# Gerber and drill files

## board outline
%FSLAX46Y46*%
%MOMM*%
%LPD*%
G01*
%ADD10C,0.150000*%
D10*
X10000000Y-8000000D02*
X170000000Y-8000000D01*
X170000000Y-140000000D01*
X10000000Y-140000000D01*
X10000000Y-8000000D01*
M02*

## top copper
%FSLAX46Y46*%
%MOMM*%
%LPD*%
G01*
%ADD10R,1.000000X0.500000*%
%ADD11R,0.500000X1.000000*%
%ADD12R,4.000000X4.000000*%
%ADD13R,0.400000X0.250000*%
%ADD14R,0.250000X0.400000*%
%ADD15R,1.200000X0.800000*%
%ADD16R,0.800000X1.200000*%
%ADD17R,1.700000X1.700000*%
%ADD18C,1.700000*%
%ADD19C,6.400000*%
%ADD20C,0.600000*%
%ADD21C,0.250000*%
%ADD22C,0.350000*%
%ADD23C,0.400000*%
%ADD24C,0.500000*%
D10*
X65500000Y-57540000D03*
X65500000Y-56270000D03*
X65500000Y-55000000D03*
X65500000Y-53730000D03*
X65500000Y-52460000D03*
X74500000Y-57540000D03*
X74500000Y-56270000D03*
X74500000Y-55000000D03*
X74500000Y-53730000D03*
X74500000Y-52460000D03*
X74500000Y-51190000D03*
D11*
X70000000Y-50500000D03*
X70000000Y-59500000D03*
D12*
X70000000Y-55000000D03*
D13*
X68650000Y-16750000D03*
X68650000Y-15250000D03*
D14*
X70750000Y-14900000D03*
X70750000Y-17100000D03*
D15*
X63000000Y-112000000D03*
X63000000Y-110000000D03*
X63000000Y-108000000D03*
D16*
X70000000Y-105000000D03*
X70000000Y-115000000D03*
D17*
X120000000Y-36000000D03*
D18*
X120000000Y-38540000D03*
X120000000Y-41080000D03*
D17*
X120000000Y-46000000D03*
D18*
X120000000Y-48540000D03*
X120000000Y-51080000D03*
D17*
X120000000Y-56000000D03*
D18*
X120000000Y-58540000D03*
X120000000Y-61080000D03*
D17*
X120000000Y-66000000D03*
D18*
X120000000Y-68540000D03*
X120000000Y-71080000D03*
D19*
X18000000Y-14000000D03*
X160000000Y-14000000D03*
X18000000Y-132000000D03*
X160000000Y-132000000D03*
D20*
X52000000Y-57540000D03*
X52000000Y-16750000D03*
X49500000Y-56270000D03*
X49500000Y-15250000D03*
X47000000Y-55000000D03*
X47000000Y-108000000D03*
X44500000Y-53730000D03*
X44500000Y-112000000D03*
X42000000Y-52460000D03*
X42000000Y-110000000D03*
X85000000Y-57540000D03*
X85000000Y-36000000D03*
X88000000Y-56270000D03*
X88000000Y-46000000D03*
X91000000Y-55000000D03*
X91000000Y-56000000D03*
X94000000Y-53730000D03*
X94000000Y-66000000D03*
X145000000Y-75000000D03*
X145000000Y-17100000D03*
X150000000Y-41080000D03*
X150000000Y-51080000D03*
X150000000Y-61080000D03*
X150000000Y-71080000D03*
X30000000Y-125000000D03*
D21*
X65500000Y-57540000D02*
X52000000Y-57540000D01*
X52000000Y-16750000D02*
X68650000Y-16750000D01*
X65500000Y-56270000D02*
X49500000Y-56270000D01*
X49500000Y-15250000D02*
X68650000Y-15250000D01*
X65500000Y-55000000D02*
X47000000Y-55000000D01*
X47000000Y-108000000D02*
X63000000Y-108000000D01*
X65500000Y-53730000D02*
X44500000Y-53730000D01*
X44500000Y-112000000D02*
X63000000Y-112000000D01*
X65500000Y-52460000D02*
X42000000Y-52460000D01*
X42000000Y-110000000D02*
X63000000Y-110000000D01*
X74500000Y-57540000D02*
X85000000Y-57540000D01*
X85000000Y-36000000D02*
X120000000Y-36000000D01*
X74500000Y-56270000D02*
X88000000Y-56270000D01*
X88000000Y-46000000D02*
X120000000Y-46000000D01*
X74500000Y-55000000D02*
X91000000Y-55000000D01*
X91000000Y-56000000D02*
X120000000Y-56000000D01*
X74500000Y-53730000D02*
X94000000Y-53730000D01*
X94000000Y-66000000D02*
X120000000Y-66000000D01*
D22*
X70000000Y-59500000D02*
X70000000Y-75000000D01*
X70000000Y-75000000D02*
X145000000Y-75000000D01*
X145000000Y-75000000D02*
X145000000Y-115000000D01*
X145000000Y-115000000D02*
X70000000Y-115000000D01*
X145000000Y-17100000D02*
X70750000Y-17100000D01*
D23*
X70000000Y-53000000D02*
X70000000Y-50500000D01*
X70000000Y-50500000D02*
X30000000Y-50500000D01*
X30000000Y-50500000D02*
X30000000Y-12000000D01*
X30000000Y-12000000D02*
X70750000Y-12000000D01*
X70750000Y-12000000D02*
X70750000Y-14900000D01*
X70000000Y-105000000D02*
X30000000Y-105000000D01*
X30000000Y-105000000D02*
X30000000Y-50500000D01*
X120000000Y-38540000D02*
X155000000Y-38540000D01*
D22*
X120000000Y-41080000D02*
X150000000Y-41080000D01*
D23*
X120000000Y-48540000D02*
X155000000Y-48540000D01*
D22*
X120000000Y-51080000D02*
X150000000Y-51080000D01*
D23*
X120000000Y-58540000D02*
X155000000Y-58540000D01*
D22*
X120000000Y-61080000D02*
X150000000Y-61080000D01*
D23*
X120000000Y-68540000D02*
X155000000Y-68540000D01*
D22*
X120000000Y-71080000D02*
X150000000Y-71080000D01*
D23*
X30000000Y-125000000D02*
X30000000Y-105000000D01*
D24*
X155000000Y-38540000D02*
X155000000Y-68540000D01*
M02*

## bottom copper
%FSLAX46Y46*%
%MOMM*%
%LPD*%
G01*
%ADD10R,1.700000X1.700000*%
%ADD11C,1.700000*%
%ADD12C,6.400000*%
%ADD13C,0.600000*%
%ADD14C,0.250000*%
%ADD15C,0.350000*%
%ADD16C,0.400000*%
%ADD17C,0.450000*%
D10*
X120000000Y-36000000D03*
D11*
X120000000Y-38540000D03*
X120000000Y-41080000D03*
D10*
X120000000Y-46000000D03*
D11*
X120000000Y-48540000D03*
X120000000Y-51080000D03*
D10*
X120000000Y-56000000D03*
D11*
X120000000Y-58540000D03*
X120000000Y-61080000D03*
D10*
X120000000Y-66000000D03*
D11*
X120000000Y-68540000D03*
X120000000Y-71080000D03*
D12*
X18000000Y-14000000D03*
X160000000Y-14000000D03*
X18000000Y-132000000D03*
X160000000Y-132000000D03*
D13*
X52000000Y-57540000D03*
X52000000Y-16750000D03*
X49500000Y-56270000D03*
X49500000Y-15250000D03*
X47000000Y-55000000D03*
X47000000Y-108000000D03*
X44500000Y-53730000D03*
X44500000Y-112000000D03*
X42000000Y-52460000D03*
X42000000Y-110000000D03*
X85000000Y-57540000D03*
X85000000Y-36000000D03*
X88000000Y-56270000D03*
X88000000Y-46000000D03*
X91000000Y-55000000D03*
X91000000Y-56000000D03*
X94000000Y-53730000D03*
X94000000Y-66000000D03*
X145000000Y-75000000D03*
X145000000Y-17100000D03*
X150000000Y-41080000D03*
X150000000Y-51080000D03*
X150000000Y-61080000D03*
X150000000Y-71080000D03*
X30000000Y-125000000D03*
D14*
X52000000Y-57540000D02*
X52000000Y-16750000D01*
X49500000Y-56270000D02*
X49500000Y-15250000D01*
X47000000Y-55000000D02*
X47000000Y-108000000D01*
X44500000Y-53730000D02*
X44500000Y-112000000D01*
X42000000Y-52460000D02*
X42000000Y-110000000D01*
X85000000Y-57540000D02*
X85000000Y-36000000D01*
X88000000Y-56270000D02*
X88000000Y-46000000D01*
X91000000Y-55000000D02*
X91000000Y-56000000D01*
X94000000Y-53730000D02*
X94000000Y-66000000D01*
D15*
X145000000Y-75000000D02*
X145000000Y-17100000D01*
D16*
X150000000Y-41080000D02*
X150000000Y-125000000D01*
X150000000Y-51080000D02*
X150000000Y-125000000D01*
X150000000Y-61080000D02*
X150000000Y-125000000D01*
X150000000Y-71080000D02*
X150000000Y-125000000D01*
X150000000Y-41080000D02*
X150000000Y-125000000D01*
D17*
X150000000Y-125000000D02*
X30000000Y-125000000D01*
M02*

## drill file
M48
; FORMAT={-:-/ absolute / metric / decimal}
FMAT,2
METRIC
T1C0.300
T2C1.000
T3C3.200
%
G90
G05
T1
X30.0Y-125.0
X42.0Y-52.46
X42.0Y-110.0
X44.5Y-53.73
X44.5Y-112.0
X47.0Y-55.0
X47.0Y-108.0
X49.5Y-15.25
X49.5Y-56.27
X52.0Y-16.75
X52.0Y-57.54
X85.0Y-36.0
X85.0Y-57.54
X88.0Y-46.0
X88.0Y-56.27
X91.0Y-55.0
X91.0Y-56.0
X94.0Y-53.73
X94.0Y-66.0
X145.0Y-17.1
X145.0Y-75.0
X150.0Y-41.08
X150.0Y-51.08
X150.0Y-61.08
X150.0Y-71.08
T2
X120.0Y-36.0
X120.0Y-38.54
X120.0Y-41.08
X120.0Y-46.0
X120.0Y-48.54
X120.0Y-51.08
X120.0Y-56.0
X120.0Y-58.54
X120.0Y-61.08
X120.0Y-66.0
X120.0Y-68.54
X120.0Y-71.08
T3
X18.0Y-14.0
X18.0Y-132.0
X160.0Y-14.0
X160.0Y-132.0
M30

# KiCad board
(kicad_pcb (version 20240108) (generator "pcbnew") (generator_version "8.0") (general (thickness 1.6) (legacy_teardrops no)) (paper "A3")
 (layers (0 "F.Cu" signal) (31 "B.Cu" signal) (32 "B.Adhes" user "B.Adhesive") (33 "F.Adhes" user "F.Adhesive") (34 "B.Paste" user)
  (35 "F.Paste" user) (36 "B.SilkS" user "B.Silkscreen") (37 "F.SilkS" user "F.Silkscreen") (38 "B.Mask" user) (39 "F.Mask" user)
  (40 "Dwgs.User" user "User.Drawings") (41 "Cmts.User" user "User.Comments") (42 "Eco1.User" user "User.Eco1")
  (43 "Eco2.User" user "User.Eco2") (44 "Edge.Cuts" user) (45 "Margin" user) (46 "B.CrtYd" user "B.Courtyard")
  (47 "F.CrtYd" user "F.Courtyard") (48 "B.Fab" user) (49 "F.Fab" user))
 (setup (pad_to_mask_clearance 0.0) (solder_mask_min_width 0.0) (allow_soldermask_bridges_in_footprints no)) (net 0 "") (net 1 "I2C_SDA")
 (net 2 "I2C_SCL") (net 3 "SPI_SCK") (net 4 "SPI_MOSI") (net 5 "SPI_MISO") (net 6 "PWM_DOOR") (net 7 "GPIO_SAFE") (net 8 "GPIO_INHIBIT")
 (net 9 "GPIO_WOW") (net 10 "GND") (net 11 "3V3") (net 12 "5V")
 (gr_rect (start 10 8) (end 170 140) (stroke (width 0.15) (type solid)) (fill none) (layer "Edge.Cuts"))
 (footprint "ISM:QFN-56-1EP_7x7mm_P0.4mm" (layer "F.Cu") (at 70 55)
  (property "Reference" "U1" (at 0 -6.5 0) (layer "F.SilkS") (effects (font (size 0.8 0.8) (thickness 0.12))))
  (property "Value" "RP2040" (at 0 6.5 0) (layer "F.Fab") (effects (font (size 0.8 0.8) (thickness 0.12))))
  (pad "1" smd rect (at -4.5 2.54) (size 1.0 0.5) (layers "F.Cu" "F.Paste" "F.Mask") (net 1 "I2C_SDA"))
  (pad "2" smd rect (at -4.5 1.27) (size 1.0 0.5) (layers "F.Cu" "F.Paste" "F.Mask") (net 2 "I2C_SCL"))
  (pad "3" smd rect (at -4.5 0) (size 1.0 0.5) (layers "F.Cu" "F.Paste" "F.Mask") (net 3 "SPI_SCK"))
  (pad "4" smd rect (at -4.5 -1.27) (size 1.0 0.5) (layers "F.Cu" "F.Paste" "F.Mask") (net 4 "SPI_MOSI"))
  (pad "5" smd rect (at -4.5 -2.54) (size 1.0 0.5) (layers "F.Cu" "F.Paste" "F.Mask") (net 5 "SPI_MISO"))
  (pad "6" smd rect (at 4.5 2.54) (size 1.0 0.5) (layers "F.Cu" "F.Paste" "F.Mask") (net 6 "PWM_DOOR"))
  (pad "7" smd rect (at 4.5 1.27) (size 1.0 0.5) (layers "F.Cu" "F.Paste" "F.Mask") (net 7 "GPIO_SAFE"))
  (pad "8" smd rect (at 4.5 0) (size 1.0 0.5) (layers "F.Cu" "F.Paste" "F.Mask") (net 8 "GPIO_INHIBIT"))
  (pad "9" smd rect (at 4.5 -1.27) (size 1.0 0.5) (layers "F.Cu" "F.Paste" "F.Mask") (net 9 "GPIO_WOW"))
  (pad "12" smd rect (at 4.5 -2.54) (size 1.0 0.5) (layers "F.Cu" "F.Paste" "F.Mask"))
  (pad "13" smd rect (at 4.5 -3.81) (size 1.0 0.5) (layers "F.Cu" "F.Paste" "F.Mask"))
  (pad "10" smd rect (at 0 -4.5) (size 0.5 1.0) (layers "F.Cu" "F.Paste" "F.Mask") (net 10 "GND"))
  (pad "11" smd rect (at 0 4.5) (size 0.5 1.0) (layers "F.Cu" "F.Paste" "F.Mask") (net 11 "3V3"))
  (pad "EP" smd rect (at 0 0) (size 4 4) (layers "F.Cu" "F.Paste" "F.Mask") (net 10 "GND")))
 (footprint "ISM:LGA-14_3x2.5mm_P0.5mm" (layer "F.Cu") (at 70 16)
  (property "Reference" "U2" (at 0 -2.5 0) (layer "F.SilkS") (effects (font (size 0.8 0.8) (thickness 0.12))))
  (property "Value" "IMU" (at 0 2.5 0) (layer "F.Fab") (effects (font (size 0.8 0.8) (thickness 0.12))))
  (pad "1" smd rect (at -1.35 0.75) (size 0.4 0.25) (layers "F.Cu" "F.Paste" "F.Mask") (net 1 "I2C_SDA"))
  (pad "2" smd rect (at -1.35 -0.75) (size 0.4 0.25) (layers "F.Cu" "F.Paste" "F.Mask") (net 2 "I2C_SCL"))
  (pad "3" smd rect (at 0.75 -1.1) (size 0.25 0.4) (layers "F.Cu" "F.Paste" "F.Mask") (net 10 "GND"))
  (pad "4" smd rect (at 0.75 1.1) (size 0.25 0.4) (layers "F.Cu" "F.Paste" "F.Mask") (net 11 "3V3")))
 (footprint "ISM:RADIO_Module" (layer "F.Cu") (at 70 110)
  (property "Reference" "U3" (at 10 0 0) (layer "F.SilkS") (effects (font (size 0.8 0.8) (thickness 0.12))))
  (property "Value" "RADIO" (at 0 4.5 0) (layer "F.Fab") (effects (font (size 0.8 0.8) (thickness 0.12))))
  (pad "1" smd rect (at -7 2) (size 1.2 0.8) (layers "F.Cu" "F.Paste" "F.Mask") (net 4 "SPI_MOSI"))
  (pad "2" smd rect (at -7 0) (size 1.2 0.8) (layers "F.Cu" "F.Paste" "F.Mask") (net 5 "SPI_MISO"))
  (pad "3" smd rect (at -7 -2) (size 1.2 0.8) (layers "F.Cu" "F.Paste" "F.Mask") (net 3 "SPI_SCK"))
  (pad "4" smd rect (at 0 -5) (size 0.8 1.2) (layers "F.Cu" "F.Paste" "F.Mask") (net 10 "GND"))
  (pad "5" smd rect (at 0 5) (size 0.8 1.2) (layers "F.Cu" "F.Paste" "F.Mask") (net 11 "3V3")))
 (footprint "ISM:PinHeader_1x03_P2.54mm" (layer "F.Cu") (at 120 36)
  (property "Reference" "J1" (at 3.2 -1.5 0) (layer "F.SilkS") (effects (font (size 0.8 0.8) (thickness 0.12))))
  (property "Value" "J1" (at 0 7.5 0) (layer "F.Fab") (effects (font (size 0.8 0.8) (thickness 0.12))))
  (pad "1" thru_hole rect (at 0 0) (size 1.7 1.7) (drill 1.0) (layers "*.Cu" "*.Mask") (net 6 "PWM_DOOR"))
  (pad "2" thru_hole circle (at 0 2.54) (size 1.7 1.7) (drill 1.0) (layers "*.Cu" "*.Mask") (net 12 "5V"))
  (pad "3" thru_hole circle (at 0 5.08) (size 1.7 1.7) (drill 1.0) (layers "*.Cu" "*.Mask") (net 10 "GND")))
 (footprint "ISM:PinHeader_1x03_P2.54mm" (layer "F.Cu") (at 120 46)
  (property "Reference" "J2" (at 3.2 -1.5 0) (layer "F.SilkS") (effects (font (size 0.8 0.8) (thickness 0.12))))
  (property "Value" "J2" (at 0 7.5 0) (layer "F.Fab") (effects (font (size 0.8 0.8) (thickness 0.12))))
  (pad "1" thru_hole rect (at 0 0) (size 1.7 1.7) (drill 1.0) (layers "*.Cu" "*.Mask") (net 7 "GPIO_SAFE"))
  (pad "2" thru_hole circle (at 0 2.54) (size 1.7 1.7) (drill 1.0) (layers "*.Cu" "*.Mask") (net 12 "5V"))
  (pad "3" thru_hole circle (at 0 5.08) (size 1.7 1.7) (drill 1.0) (layers "*.Cu" "*.Mask") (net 10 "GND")))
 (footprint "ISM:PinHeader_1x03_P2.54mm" (layer "F.Cu") (at 120 56)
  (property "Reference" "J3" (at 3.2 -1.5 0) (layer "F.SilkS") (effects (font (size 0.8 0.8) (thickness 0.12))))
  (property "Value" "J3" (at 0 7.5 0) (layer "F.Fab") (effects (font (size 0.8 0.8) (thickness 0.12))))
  (pad "1" thru_hole rect (at 0 0) (size 1.7 1.7) (drill 1.0) (layers "*.Cu" "*.Mask") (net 8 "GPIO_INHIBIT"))
  (pad "2" thru_hole circle (at 0 2.54) (size 1.7 1.7) (drill 1.0) (layers "*.Cu" "*.Mask") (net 12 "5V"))
  (pad "3" thru_hole circle (at 0 5.08) (size 1.7 1.7) (drill 1.0) (layers "*.Cu" "*.Mask") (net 10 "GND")))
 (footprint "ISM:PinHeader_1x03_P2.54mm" (layer "F.Cu") (at 120 66)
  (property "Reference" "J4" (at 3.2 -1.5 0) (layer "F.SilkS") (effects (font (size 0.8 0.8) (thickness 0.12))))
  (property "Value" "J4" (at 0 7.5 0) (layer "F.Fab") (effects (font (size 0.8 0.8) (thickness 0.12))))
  (pad "1" thru_hole rect (at 0 0) (size 1.7 1.7) (drill 1.0) (layers "*.Cu" "*.Mask") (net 9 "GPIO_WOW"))
  (pad "2" thru_hole circle (at 0 2.54) (size 1.7 1.7) (drill 1.0) (layers "*.Cu" "*.Mask") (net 12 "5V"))
  (pad "3" thru_hole circle (at 0 5.08) (size 1.7 1.7) (drill 1.0) (layers "*.Cu" "*.Mask") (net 10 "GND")))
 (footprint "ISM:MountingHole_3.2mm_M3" (layer "F.Cu") (at 18 14)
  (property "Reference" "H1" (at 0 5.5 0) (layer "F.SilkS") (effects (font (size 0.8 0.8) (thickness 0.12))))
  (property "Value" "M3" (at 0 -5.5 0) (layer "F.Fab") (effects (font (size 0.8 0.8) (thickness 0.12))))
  (pad "" thru_hole circle (at 0 0) (size 6.4 6.4) (drill 3.2) (layers "*.Cu" "*.Mask")))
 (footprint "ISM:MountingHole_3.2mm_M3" (layer "F.Cu") (at 160 14)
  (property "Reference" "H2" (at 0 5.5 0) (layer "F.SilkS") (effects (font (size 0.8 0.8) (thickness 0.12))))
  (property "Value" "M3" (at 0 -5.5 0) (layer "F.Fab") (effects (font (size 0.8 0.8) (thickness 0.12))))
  (pad "" thru_hole circle (at 0 0) (size 6.4 6.4) (drill 3.2) (layers "*.Cu" "*.Mask")))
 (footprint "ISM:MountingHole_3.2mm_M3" (layer "F.Cu") (at 18 132)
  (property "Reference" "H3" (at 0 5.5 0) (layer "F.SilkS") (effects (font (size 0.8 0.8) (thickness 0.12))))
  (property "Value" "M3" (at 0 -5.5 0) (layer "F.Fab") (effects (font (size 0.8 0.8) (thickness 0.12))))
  (pad "" thru_hole circle (at 0 0) (size 6.4 6.4) (drill 3.2) (layers "*.Cu" "*.Mask")))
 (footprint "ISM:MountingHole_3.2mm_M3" (layer "F.Cu") (at 160 132)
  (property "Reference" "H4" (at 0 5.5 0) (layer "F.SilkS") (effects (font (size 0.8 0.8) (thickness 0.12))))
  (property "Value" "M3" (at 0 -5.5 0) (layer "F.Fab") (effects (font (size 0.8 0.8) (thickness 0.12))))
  (pad "" thru_hole circle (at 0 0) (size 6.4 6.4) (drill 3.2) (layers "*.Cu" "*.Mask")))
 (segment (start 65.5 57.54) (end 52.0 57.54) (width 0.25) (layer "F.Cu") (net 1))
 (segment (start 52.0 57.54) (end 52.0 16.75) (width 0.25) (layer "B.Cu") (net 1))
 (segment (start 52.0 16.75) (end 68.65 16.75) (width 0.25) (layer "F.Cu") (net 1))
 (segment (start 65.5 56.27) (end 49.5 56.27) (width 0.25) (layer "F.Cu") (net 2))
 (segment (start 49.5 56.27) (end 49.5 15.25) (width 0.25) (layer "B.Cu") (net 2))
 (segment (start 49.5 15.25) (end 68.65 15.25) (width 0.25) (layer "F.Cu") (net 2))
 (segment (start 65.5 55) (end 47.0 55) (width 0.25) (layer "F.Cu") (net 3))
 (segment (start 47.0 55) (end 47.0 108) (width 0.25) (layer "B.Cu") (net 3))
 (segment (start 47.0 108) (end 63 108) (width 0.25) (layer "F.Cu") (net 3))
 (segment (start 65.5 53.73) (end 44.5 53.73) (width 0.25) (layer "F.Cu") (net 4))
 (segment (start 44.5 53.73) (end 44.5 112) (width 0.25) (layer "B.Cu") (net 4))
 (segment (start 44.5 112) (end 63 112) (width 0.25) (layer "F.Cu") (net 4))
 (segment (start 65.5 52.46) (end 42.0 52.46) (width 0.25) (layer "F.Cu") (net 5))
 (segment (start 42.0 52.46) (end 42.0 110) (width 0.25) (layer "B.Cu") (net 5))
 (segment (start 42.0 110) (end 63 110) (width 0.25) (layer "F.Cu") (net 5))
 (segment (start 74.5 57.54) (end 85 57.54) (width 0.25) (layer "F.Cu") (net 6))
 (segment (start 85 57.54) (end 85 36) (width 0.25) (layer "B.Cu") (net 6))
 (segment (start 85 36) (end 120 36) (width 0.25) (layer "F.Cu") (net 6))
 (segment (start 74.5 56.27) (end 88 56.27) (width 0.25) (layer "F.Cu") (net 7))
 (segment (start 88 56.27) (end 88 46) (width 0.25) (layer "B.Cu") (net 7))
 (segment (start 88 46) (end 120 46) (width 0.25) (layer "F.Cu") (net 7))
 (segment (start 74.5 55) (end 91 55) (width 0.25) (layer "F.Cu") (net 8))
 (segment (start 91 55) (end 91 56) (width 0.25) (layer "B.Cu") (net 8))
 (segment (start 91 56) (end 120 56) (width 0.25) (layer "F.Cu") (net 8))
 (segment (start 74.5 53.73) (end 94 53.73) (width 0.25) (layer "F.Cu") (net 9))
 (segment (start 94 53.73) (end 94 66) (width 0.25) (layer "B.Cu") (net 9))
 (segment (start 94 66) (end 120 66) (width 0.25) (layer "F.Cu") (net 9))
 (segment (start 70 59.5) (end 70 75) (width 0.35) (layer "F.Cu") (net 11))
 (segment (start 70 75) (end 145 75) (width 0.35) (layer "F.Cu") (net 11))
 (segment (start 145 75) (end 145 115) (width 0.35) (layer "F.Cu") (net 11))
 (segment (start 145 115) (end 70 115) (width 0.35) (layer "F.Cu") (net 11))
 (segment (start 145 75) (end 145 17.1) (width 0.35) (layer "B.Cu") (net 11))
 (segment (start 145 17.1) (end 70.75 17.1) (width 0.35) (layer "F.Cu") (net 11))
 (segment (start 70 53) (end 70 50.5) (width 0.4) (layer "F.Cu") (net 10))
 (segment (start 70 50.5) (end 30 50.5) (width 0.4) (layer "F.Cu") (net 10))
 (segment (start 30 50.5) (end 30 12) (width 0.4) (layer "F.Cu") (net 10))
 (segment (start 30 12) (end 70.75 12) (width 0.4) (layer "F.Cu") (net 10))
 (segment (start 70.75 12) (end 70.75 14.9) (width 0.4) (layer "F.Cu") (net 10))
 (segment (start 70 105) (end 30 105) (width 0.4) (layer "F.Cu") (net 10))
 (segment (start 30 105) (end 30 50.5) (width 0.4) (layer "F.Cu") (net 10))
 (segment (start 120 38.54) (end 155 38.54) (width 0.4) (layer "F.Cu") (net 12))
 (segment (start 120 41.08) (end 150 41.08) (width 0.35) (layer "F.Cu") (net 10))
 (segment (start 150 41.08) (end 150 125) (width 0.4) (layer "B.Cu") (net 10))
 (segment (start 120 48.54) (end 155 48.54) (width 0.4) (layer "F.Cu") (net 12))
 (segment (start 120 51.08) (end 150 51.08) (width 0.35) (layer "F.Cu") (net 10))
 (segment (start 150 51.08) (end 150 125) (width 0.4) (layer "B.Cu") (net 10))
 (segment (start 120 58.54) (end 155 58.54) (width 0.4) (layer "F.Cu") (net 12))
 (segment (start 120 61.08) (end 150 61.08) (width 0.35) (layer "F.Cu") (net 10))
 (segment (start 150 61.08) (end 150 125) (width 0.4) (layer "B.Cu") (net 10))
 (segment (start 120 68.54) (end 155 68.54) (width 0.4) (layer "F.Cu") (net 12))
 (segment (start 120 71.08) (end 150 71.08) (width 0.35) (layer "F.Cu") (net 10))
 (segment (start 150 71.08) (end 150 125) (width 0.4) (layer "B.Cu") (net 10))
 (segment (start 150 41.08) (end 150 125) (width 0.4) (layer "B.Cu") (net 10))
 (segment (start 150 125) (end 30 125) (width 0.45) (layer "B.Cu") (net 10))
 (segment (start 30 125) (end 30 105) (width 0.4) (layer "F.Cu") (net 10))
 (segment (start 155 38.54) (end 155 68.54) (width 0.5) (layer "F.Cu") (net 12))
 (via (at 52.0 57.54) (size 0.6) (drill 0.3) (layers "F.Cu" "B.Cu") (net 1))
 (via (at 52.0 16.75) (size 0.6) (drill 0.3) (layers "F.Cu" "B.Cu") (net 1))
 (via (at 49.5 56.27) (size 0.6) (drill 0.3) (layers "F.Cu" "B.Cu") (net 2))
 (via (at 49.5 15.25) (size 0.6) (drill 0.3) (layers "F.Cu" "B.Cu") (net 2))
 (via (at 47.0 55) (size 0.6) (drill 0.3) (layers "F.Cu" "B.Cu") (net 3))
 (via (at 47.0 108) (size 0.6) (drill 0.3) (layers "F.Cu" "B.Cu") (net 3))
 (via (at 44.5 53.73) (size 0.6) (drill 0.3) (layers "F.Cu" "B.Cu") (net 4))
 (via (at 44.5 112) (size 0.6) (drill 0.3) (layers "F.Cu" "B.Cu") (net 4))
 (via (at 42.0 52.46) (size 0.6) (drill 0.3) (layers "F.Cu" "B.Cu") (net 5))
 (via (at 42.0 110) (size 0.6) (drill 0.3) (layers "F.Cu" "B.Cu") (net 5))
 (via (at 85 57.54) (size 0.6) (drill 0.3) (layers "F.Cu" "B.Cu") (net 6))
 (via (at 85 36) (size 0.6) (drill 0.3) (layers "F.Cu" "B.Cu") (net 6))
 (via (at 88 56.27) (size 0.6) (drill 0.3) (layers "F.Cu" "B.Cu") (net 7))
 (via (at 88 46) (size 0.6) (drill 0.3) (layers "F.Cu" "B.Cu") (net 7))
 (via (at 91 55) (size 0.6) (drill 0.3) (layers "F.Cu" "B.Cu") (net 8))
 (via (at 91 56) (size 0.6) (drill 0.3) (layers "F.Cu" "B.Cu") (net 8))
 (via (at 94 53.73) (size 0.6) (drill 0.3) (layers "F.Cu" "B.Cu") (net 9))
 (via (at 94 66) (size 0.6) (drill 0.3) (layers "F.Cu" "B.Cu") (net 9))
 (via (at 145 75) (size 0.6) (drill 0.3) (layers "F.Cu" "B.Cu") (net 11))
 (via (at 145 17.1) (size 0.6) (drill 0.3) (layers "F.Cu" "B.Cu") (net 11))
 (via (at 150 41.08) (size 0.6) (drill 0.3) (layers "F.Cu" "B.Cu") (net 10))
 (via (at 150 51.08) (size 0.6) (drill 0.3) (layers "F.Cu" "B.Cu") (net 10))
 (via (at 150 61.08) (size 0.6) (drill 0.3) (layers "F.Cu" "B.Cu") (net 10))
 (via (at 150 71.08) (size 0.6) (drill 0.3) (layers "F.Cu" "B.Cu") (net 10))
 (via (at 30 125) (size 0.6) (drill 0.3) (layers "F.Cu" "B.Cu") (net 10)))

